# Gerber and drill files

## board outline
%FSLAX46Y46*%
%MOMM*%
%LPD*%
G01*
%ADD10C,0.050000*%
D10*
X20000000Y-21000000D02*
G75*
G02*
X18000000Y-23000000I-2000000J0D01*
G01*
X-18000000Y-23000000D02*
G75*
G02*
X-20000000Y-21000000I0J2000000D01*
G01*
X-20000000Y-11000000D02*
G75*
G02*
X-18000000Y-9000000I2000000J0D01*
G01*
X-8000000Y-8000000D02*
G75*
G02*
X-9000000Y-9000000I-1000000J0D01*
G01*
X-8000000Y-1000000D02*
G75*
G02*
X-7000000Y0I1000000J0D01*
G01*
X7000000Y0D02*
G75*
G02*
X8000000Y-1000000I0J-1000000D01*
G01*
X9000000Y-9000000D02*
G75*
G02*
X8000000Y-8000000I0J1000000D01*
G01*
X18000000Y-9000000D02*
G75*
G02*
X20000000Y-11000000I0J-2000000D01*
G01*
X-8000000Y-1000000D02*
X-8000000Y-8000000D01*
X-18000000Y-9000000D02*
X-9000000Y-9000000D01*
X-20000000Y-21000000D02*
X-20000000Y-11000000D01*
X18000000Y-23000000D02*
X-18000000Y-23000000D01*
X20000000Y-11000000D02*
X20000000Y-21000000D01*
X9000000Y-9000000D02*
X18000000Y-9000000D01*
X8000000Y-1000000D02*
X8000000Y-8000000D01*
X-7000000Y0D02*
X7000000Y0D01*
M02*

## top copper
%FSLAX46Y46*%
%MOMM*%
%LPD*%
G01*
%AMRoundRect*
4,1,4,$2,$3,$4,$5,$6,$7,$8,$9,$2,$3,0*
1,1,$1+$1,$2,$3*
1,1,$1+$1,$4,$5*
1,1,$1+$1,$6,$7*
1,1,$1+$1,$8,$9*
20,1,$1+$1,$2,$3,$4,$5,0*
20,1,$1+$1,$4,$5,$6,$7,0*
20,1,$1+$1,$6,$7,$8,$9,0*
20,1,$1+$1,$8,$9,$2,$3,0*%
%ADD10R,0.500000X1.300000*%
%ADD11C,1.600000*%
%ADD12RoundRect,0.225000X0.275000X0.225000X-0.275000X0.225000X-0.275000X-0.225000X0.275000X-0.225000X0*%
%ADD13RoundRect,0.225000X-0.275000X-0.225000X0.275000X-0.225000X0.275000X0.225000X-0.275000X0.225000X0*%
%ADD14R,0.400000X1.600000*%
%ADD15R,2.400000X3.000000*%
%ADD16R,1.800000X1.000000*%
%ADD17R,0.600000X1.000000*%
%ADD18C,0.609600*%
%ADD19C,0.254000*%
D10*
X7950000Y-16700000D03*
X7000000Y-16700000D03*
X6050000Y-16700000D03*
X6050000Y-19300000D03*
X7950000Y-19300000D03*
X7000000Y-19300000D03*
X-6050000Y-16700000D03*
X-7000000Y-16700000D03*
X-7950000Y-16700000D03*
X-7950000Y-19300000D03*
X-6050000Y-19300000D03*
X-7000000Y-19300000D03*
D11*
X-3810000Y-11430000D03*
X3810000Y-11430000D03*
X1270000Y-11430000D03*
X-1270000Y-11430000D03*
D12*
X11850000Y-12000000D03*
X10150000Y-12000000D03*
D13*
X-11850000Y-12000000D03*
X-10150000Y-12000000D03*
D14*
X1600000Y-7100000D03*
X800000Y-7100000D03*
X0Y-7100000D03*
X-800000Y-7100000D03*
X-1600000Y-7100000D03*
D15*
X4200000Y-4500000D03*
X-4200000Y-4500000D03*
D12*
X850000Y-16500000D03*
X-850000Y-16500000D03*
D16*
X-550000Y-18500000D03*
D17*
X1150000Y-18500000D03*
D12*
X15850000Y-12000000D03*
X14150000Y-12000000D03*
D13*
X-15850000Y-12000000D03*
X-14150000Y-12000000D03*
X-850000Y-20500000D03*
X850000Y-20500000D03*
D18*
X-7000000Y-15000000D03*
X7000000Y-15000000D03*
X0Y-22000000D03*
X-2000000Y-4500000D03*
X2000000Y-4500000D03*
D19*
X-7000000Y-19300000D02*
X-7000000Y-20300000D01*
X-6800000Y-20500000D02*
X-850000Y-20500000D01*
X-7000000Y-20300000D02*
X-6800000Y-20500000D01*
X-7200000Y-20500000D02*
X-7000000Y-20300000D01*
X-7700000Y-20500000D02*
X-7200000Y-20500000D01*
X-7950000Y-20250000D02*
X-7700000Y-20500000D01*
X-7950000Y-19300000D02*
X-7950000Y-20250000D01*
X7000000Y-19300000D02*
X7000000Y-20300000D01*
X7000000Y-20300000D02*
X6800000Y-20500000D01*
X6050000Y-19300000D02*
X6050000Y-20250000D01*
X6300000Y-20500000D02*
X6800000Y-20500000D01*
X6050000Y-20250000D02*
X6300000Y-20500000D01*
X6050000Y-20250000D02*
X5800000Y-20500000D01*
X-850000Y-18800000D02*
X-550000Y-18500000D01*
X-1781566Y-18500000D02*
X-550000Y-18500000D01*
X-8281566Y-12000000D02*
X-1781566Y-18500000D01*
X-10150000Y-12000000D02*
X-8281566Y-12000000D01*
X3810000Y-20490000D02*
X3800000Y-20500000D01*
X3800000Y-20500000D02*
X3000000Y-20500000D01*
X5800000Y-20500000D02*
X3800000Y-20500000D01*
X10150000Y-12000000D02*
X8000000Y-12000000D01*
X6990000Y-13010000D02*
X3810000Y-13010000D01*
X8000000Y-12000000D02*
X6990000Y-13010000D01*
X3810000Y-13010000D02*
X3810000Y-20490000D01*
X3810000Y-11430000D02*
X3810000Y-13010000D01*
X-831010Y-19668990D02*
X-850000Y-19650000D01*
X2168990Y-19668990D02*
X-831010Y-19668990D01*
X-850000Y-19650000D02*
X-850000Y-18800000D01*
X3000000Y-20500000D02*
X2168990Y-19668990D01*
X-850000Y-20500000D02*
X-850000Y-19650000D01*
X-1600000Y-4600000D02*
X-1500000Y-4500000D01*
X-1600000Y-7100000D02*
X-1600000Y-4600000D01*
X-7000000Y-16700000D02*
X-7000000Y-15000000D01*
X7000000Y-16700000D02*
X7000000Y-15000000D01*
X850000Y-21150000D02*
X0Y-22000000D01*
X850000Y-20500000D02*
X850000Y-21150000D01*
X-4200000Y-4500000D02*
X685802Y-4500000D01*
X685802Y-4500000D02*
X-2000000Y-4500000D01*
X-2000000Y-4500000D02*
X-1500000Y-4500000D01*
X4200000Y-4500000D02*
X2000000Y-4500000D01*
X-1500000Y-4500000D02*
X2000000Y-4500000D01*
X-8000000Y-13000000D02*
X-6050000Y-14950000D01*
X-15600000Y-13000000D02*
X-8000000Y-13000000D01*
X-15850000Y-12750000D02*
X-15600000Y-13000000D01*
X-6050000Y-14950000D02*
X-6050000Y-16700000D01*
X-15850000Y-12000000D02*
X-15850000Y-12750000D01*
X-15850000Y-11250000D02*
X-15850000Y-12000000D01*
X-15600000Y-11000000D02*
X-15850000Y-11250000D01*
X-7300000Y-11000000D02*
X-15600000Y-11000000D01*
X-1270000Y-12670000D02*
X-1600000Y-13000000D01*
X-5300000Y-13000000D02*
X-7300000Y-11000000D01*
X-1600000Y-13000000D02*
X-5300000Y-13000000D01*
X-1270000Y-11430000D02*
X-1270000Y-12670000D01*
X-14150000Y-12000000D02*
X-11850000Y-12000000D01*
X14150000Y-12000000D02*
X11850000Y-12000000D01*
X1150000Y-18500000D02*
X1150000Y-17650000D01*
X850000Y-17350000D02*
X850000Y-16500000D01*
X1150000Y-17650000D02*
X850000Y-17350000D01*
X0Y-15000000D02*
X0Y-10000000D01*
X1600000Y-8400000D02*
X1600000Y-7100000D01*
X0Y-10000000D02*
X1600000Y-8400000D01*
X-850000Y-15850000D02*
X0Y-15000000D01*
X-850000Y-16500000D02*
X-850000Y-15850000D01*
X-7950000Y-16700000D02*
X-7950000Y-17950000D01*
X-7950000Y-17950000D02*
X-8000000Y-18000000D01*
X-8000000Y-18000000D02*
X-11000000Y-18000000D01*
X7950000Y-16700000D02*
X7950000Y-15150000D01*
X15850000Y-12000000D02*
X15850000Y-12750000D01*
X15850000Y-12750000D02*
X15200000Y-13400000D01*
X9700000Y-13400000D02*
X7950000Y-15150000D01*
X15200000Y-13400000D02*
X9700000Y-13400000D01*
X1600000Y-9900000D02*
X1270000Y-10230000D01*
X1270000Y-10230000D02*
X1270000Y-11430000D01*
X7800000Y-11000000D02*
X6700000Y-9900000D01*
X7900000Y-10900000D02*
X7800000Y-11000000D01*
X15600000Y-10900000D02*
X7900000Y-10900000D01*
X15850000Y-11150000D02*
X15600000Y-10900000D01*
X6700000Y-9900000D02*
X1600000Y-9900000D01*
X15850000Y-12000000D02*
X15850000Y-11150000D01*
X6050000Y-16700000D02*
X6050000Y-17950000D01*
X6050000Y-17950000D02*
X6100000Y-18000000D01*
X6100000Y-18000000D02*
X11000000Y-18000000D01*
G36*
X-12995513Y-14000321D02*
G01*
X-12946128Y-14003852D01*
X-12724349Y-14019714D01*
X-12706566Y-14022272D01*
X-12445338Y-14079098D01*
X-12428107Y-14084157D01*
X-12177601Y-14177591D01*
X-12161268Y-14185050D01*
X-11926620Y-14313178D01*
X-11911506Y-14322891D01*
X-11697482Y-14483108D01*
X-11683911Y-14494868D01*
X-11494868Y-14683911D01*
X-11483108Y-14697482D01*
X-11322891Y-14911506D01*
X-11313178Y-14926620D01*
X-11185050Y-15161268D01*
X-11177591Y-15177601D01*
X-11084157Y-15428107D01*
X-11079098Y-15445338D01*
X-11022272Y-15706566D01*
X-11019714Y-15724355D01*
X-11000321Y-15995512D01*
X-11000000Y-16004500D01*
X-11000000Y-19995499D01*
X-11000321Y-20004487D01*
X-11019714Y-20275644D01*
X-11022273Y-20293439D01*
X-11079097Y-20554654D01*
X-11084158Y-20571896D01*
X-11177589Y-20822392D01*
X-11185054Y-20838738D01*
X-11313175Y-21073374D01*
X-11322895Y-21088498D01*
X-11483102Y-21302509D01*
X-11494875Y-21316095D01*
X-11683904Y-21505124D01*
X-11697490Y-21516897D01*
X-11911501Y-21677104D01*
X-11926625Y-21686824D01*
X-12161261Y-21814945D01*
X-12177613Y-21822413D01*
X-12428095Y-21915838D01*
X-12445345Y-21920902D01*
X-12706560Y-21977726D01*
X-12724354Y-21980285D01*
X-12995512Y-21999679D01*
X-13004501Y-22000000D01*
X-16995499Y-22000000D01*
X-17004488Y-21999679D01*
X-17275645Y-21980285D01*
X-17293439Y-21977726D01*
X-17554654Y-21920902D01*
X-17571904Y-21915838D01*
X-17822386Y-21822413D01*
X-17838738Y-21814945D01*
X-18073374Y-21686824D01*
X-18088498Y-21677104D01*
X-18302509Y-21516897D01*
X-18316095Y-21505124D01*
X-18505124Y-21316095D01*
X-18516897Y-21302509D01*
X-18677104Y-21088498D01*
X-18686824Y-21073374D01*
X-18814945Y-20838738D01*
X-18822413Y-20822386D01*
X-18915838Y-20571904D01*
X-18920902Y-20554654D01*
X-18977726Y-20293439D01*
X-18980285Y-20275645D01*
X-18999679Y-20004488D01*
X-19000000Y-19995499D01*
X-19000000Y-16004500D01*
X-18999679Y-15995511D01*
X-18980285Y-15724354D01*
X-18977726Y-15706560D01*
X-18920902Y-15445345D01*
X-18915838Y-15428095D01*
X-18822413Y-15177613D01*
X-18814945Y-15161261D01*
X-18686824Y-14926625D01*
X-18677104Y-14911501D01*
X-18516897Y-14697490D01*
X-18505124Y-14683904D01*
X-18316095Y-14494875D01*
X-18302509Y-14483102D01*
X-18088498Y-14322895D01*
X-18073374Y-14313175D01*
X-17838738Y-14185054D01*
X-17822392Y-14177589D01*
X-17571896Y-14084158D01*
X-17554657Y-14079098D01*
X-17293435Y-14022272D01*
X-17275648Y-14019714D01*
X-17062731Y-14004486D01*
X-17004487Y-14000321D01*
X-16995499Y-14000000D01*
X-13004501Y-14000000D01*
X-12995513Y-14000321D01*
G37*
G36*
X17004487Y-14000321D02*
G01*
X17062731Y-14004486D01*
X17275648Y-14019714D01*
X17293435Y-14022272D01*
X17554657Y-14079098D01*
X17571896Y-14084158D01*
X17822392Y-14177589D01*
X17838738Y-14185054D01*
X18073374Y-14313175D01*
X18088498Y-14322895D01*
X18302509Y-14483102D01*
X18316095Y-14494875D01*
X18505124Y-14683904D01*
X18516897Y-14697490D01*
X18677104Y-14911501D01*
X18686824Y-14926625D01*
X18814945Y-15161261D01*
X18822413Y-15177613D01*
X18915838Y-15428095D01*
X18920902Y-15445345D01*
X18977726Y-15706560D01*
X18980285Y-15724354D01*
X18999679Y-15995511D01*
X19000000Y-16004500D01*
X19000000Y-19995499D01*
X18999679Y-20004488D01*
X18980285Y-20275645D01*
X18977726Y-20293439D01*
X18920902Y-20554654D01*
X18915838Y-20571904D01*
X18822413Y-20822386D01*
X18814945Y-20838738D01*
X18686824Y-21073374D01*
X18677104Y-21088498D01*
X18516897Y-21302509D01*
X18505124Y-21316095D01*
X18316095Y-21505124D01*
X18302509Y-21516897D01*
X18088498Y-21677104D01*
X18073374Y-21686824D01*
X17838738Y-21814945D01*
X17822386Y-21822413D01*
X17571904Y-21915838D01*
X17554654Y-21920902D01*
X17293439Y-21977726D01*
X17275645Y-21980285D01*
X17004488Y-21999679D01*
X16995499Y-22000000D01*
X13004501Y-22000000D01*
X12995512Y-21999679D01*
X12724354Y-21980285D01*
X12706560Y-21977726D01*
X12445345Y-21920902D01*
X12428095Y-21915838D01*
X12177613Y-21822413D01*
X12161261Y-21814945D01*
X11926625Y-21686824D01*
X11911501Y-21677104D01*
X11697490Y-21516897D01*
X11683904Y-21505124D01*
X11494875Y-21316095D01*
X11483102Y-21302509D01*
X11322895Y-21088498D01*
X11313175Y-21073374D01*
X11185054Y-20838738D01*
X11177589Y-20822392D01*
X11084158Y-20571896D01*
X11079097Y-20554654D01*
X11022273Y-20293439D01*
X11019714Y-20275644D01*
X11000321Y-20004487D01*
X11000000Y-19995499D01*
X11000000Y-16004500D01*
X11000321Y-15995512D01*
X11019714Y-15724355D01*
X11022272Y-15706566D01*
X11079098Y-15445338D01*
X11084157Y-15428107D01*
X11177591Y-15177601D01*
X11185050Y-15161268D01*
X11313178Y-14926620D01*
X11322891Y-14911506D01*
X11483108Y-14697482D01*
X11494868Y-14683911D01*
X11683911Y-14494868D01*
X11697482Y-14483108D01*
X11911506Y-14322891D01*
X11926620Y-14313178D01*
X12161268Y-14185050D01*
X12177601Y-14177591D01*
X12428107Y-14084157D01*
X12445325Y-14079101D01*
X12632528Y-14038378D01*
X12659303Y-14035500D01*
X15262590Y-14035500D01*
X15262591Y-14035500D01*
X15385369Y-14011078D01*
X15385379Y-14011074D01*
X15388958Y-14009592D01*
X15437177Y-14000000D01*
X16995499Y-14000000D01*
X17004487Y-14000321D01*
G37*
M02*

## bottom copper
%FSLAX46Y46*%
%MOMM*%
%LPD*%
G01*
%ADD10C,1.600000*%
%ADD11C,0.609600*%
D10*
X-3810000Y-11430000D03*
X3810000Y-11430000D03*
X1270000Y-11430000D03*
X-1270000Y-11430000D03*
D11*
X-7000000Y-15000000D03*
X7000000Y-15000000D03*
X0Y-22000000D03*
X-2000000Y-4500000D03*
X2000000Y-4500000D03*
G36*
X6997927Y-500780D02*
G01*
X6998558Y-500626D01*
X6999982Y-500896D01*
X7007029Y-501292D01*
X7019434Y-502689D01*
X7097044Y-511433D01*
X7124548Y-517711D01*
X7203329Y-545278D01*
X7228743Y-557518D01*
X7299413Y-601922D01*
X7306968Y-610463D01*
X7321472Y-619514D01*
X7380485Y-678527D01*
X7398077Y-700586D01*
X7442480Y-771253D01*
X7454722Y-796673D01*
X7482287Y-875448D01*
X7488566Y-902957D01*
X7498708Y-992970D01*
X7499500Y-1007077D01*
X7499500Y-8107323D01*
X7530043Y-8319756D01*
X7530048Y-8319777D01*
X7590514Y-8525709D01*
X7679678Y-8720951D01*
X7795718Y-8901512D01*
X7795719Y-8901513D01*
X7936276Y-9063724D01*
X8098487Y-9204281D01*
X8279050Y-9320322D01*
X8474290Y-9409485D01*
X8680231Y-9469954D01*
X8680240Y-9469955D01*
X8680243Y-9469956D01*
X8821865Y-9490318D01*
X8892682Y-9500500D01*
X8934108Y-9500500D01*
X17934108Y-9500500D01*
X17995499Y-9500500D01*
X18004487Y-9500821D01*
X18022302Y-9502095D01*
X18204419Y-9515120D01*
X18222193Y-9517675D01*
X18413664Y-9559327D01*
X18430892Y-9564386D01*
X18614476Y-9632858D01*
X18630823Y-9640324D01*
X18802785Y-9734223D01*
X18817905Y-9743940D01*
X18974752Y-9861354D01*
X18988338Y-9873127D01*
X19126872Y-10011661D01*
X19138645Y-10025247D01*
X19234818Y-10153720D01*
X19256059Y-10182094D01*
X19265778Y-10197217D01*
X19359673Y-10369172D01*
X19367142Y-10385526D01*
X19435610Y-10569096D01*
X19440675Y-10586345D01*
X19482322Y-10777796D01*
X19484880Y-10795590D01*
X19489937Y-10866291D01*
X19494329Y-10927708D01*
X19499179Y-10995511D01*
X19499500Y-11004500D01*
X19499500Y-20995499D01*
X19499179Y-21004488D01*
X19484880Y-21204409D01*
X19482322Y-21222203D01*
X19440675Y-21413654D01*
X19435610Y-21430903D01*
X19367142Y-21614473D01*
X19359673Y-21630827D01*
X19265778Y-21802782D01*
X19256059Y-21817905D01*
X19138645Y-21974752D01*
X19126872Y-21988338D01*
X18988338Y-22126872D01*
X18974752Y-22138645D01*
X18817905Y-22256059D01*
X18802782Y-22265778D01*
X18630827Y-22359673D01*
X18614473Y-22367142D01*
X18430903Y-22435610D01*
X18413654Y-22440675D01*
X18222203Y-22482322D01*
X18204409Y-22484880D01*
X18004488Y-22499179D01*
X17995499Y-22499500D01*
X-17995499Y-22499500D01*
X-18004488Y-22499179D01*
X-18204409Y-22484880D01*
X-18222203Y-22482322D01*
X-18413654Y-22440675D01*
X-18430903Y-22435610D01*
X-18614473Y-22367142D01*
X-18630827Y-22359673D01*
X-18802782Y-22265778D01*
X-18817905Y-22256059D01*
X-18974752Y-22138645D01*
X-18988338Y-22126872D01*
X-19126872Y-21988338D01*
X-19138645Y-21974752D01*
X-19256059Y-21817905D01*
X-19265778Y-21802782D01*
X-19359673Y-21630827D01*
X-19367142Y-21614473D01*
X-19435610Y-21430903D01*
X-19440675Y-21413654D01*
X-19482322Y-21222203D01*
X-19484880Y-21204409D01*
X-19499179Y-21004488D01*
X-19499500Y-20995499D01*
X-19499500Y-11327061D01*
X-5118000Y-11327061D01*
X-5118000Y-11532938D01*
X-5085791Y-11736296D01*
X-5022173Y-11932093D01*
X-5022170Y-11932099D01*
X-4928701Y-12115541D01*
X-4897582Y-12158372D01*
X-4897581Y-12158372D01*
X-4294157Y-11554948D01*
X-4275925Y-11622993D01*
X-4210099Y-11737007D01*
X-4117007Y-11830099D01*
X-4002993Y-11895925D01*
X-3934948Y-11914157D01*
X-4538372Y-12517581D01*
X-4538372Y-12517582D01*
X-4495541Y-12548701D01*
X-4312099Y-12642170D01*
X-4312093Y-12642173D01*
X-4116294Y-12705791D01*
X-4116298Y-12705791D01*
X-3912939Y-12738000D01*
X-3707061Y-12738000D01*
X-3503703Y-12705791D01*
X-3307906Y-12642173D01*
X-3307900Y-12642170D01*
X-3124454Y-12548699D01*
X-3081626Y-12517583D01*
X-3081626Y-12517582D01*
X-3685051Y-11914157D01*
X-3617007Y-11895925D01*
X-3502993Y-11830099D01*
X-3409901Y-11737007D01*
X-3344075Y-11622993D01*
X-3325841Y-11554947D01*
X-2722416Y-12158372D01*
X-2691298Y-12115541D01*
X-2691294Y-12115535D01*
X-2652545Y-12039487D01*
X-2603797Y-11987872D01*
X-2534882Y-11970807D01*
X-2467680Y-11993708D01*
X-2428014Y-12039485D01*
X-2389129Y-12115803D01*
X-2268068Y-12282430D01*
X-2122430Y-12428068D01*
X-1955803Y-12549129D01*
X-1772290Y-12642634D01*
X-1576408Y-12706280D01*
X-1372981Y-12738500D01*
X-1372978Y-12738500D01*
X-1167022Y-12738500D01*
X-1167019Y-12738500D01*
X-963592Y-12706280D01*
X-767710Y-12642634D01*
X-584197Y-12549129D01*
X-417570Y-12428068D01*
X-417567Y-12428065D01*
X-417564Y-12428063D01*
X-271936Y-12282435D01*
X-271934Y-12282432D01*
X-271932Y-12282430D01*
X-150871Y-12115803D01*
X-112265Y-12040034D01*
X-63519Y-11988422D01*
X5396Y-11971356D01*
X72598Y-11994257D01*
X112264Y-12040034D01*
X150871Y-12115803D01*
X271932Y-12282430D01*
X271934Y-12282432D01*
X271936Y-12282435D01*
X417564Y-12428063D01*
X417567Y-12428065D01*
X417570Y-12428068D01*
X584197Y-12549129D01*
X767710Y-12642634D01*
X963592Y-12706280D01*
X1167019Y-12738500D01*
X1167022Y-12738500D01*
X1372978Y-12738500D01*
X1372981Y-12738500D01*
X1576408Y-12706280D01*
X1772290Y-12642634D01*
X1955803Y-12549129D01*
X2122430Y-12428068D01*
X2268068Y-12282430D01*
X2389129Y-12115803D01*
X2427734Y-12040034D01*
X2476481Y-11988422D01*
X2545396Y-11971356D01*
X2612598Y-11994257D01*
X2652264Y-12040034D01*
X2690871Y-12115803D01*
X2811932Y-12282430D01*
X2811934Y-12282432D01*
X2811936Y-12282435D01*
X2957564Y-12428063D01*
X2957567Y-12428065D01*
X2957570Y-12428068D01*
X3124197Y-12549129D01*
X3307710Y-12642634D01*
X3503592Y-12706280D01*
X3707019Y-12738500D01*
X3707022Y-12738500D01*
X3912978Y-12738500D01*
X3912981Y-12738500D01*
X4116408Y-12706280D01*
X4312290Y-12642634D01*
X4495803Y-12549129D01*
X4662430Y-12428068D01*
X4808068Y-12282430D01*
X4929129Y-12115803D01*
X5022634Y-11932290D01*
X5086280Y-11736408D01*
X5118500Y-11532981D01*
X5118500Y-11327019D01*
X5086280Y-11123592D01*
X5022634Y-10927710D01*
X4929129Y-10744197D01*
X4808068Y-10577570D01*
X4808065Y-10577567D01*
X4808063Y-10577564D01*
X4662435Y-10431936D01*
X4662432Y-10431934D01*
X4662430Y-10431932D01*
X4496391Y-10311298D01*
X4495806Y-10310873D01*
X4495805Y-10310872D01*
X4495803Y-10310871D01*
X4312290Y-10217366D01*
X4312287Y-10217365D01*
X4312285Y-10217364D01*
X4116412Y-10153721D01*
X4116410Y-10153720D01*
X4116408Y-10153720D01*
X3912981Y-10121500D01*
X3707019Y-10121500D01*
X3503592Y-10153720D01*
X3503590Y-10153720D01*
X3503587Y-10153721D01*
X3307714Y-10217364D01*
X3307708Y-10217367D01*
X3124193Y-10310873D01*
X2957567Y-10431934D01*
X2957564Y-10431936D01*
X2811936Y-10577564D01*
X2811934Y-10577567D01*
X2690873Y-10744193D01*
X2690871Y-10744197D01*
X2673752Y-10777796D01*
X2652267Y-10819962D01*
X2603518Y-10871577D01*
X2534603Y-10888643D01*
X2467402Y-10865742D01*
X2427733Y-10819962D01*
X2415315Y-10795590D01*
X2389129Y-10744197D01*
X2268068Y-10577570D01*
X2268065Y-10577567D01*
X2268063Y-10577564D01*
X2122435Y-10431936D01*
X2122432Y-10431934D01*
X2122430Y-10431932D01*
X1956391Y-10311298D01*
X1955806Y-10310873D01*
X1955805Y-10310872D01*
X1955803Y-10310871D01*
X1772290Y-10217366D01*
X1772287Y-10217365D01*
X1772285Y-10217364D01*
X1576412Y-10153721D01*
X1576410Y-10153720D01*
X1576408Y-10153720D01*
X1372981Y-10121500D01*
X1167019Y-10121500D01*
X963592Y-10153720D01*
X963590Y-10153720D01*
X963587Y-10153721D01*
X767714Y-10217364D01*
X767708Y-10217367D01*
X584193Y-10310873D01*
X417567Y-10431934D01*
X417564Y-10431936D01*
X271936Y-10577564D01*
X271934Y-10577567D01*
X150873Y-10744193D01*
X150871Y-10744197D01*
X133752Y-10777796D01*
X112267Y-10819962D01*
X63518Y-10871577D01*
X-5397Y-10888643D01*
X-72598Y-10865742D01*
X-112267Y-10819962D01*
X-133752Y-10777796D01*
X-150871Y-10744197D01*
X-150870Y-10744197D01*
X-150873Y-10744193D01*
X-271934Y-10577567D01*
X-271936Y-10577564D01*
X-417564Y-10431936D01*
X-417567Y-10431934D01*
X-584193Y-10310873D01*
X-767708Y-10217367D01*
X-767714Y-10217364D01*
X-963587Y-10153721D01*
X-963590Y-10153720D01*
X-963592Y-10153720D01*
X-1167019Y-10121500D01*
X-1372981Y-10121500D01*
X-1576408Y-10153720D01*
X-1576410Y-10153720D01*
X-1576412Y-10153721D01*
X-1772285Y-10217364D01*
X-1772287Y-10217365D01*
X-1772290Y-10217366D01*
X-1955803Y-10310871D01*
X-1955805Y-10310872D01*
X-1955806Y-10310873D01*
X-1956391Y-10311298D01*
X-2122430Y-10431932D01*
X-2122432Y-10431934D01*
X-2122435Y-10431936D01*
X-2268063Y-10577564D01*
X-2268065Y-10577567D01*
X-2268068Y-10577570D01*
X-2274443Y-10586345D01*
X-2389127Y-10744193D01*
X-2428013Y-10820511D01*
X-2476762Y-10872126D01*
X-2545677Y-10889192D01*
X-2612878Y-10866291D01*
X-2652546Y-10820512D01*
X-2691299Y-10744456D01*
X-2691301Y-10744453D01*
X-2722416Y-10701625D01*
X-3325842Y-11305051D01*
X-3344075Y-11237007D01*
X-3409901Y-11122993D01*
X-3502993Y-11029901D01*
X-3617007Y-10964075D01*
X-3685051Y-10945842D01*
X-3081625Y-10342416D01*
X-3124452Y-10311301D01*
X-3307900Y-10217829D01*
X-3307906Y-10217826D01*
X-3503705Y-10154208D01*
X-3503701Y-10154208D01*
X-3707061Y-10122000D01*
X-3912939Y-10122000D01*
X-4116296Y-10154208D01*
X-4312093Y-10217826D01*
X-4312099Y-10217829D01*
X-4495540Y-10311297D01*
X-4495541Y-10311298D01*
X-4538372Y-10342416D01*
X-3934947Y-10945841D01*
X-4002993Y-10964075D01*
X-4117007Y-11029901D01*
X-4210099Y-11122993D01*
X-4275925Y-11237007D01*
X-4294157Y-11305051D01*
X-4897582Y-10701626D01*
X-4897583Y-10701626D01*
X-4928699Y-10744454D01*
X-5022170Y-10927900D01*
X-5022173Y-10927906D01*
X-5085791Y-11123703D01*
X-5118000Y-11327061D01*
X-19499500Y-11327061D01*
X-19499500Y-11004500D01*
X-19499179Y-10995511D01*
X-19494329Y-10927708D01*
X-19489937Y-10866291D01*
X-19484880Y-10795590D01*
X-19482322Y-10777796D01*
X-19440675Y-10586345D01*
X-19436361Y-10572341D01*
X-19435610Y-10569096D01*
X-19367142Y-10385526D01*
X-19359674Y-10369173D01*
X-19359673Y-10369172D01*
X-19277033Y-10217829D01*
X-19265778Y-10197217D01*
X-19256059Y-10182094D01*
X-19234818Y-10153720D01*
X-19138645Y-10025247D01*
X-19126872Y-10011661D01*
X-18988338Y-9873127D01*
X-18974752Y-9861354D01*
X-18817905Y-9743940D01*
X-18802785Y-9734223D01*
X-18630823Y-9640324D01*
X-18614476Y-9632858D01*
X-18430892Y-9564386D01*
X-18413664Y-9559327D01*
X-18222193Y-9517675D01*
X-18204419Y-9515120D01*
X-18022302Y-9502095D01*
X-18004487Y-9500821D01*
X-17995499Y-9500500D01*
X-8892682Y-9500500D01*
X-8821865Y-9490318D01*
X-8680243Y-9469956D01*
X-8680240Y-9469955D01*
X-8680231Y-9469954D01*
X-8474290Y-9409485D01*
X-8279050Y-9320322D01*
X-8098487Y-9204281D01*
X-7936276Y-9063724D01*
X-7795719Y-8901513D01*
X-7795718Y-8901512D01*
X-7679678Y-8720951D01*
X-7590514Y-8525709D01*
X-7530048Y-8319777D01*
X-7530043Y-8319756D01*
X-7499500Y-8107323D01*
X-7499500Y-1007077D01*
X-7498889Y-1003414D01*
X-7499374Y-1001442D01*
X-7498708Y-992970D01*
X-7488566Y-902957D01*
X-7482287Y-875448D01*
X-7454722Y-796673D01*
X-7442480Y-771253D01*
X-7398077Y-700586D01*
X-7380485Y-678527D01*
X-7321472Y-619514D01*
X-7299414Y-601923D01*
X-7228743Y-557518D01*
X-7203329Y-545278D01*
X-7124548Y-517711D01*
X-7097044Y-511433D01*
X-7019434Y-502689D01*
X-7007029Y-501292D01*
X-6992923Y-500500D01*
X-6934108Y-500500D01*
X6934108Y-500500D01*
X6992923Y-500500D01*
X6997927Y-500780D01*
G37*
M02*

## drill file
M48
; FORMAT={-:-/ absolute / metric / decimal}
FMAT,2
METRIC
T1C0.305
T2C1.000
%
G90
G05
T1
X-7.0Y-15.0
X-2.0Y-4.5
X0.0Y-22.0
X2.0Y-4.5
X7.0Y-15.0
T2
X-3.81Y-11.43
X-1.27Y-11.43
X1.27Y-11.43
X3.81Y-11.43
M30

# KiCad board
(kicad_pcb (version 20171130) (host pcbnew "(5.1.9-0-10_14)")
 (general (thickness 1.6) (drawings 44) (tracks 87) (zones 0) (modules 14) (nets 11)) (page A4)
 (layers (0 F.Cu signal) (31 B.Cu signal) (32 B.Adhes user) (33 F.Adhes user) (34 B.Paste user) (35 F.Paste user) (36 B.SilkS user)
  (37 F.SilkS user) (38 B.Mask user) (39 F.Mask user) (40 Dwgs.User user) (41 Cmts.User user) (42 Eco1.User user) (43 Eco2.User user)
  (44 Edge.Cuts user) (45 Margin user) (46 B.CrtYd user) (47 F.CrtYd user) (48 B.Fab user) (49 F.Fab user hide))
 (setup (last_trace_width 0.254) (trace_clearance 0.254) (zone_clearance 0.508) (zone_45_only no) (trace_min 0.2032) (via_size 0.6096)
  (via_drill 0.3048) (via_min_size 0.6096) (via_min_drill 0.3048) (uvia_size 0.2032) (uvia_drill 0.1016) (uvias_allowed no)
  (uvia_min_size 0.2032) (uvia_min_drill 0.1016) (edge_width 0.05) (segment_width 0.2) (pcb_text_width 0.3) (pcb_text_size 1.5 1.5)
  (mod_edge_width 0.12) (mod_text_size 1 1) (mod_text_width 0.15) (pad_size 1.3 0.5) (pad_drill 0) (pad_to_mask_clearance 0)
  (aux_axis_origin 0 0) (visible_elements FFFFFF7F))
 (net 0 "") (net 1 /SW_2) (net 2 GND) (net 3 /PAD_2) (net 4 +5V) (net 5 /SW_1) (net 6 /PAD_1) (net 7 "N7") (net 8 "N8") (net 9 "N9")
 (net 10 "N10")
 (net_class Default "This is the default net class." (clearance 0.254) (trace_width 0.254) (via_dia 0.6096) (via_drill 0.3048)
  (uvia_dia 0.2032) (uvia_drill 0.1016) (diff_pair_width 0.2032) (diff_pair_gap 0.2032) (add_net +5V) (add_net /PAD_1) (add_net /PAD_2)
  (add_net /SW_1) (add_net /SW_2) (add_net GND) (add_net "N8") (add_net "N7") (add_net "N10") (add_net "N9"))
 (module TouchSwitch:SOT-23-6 (layer F.Cu) (at 7 18 270)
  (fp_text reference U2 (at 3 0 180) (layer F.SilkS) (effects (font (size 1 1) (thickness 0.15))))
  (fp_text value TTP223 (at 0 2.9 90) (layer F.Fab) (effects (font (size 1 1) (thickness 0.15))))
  (pad 1 smd rect (at -1.3 -0.95 270) (size 1.3 0.5) (layers F.Cu F.Paste F.Mask) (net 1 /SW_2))
  (pad 2 smd rect (at -1.3 0 270) (size 1.3 0.5) (layers F.Cu F.Paste F.Mask) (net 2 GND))
  (pad 3 smd rect (at -1.3 0.95 270) (size 1.3 0.5) (layers F.Cu F.Paste F.Mask) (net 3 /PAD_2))
  (pad 4 smd rect (at 1.3 0.95 270) (size 1.3 0.5) (layers F.Cu F.Paste F.Mask) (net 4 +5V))
  (pad 6 smd rect (at 1.3 -0.95 270) (size 1.3 0.5) (layers F.Cu F.Paste F.Mask))
  (pad 5 smd rect (at 1.3 0 270) (size 1.3 0.5) (layers F.Cu F.Paste F.Mask) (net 4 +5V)))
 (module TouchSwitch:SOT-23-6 (layer F.Cu) (at -7 18 270)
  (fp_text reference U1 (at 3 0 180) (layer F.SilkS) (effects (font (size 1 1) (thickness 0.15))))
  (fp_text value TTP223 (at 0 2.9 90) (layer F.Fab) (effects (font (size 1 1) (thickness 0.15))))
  (pad 1 smd rect (at -1.3 -0.95 270) (size 1.3 0.5) (layers F.Cu F.Paste F.Mask) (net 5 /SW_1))
  (pad 2 smd rect (at -1.3 0 270) (size 1.3 0.5) (layers F.Cu F.Paste F.Mask) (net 2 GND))
  (pad 3 smd rect (at -1.3 0.95 270) (size 1.3 0.5) (layers F.Cu F.Paste F.Mask) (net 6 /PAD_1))
  (pad 4 smd rect (at 1.3 0.95 270) (size 1.3 0.5) (layers F.Cu F.Paste F.Mask) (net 4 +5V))
  (pad 6 smd rect (at 1.3 -0.95 270) (size 1.3 0.5) (layers F.Cu F.Paste F.Mask))
  (pad 5 smd rect (at 1.3 0 270) (size 1.3 0.5) (layers F.Cu F.Paste F.Mask) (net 4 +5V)))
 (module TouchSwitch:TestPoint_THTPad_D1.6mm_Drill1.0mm (layer F.Cu) (at -3.81 11.43)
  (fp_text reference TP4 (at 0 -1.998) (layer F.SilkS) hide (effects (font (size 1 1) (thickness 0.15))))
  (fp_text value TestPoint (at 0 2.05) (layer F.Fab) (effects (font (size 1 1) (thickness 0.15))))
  (pad 1 thru_hole circle (at 0 0) (size 1.6 1.6) (drill 1) (layers *.Cu *.Mask) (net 2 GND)))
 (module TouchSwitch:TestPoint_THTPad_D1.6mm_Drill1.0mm (layer F.Cu) (at 3.81 11.43)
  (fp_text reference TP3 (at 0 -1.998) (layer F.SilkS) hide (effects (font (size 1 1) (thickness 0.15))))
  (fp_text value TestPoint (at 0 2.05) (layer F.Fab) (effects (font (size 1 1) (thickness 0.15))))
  (pad 1 thru_hole circle (at 0 0) (size 1.6 1.6) (drill 1) (layers *.Cu *.Mask) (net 4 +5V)))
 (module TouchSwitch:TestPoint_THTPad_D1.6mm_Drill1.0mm (layer F.Cu) (at 1.27 11.43)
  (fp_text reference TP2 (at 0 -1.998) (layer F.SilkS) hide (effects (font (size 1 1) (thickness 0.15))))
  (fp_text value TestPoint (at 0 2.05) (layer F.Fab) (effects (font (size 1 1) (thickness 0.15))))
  (pad 1 thru_hole circle (at 0 0) (size 1.6 1.6) (drill 1) (layers *.Cu *.Mask) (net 1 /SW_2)))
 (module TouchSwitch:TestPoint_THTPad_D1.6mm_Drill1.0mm (layer F.Cu) (at -1.27 11.43)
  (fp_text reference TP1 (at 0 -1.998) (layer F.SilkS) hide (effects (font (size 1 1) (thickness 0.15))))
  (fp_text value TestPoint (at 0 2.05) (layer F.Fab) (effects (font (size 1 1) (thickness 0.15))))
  (pad 1 thru_hole circle (at 0 0) (size 1.6 1.6) (drill 1) (layers *.Cu *.Mask) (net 5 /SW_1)))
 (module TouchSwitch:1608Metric (layer F.Cu) (at 11 12 180)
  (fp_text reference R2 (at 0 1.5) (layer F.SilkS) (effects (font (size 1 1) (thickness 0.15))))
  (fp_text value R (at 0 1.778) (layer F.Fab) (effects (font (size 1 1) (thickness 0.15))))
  (pad 1 smd roundrect (at -0.85 0 180) (size 1 0.9) (layers F.Cu F.Paste F.Mask) (roundrect_rratio 0.25) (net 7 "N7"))
  (pad 2 smd roundrect (at 0.85 0 180) (size 1 0.9) (layers F.Cu F.Paste F.Mask) (roundrect_rratio 0.25) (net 4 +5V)))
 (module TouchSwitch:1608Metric (layer F.Cu) (at -11 12)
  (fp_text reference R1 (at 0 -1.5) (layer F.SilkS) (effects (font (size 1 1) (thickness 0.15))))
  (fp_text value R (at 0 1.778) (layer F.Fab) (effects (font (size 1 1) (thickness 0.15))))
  (pad 1 smd roundrect (at -0.85 0) (size 1 0.9) (layers F.Cu F.Paste F.Mask) (roundrect_rratio 0.25) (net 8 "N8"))
  (pad 2 smd roundrect (at 0.85 0) (size 1 0.9) (layers F.Cu F.Paste F.Mask) (roundrect_rratio 0.25) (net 4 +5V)))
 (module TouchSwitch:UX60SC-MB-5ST (layer F.Cu) (at 0 0 180)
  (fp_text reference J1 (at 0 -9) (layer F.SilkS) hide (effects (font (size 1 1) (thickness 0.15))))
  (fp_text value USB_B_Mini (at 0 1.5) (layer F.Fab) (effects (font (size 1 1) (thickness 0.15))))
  (pad 1 smd rect (at -1.6 -7.1 180) (size 0.4 1.6) (layers F.Cu F.Paste F.Mask) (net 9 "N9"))
  (pad 2 smd rect (at -0.8 -7.1 180) (size 0.4 1.6) (layers F.Cu F.Paste F.Mask))
  (pad 3 smd rect (at 0 -7.1 180) (size 0.4 1.6) (layers F.Cu F.Paste F.Mask))
  (pad 4 smd rect (at 0.8 -7.1 180) (size 0.4 1.6) (layers F.Cu F.Paste F.Mask))
  (pad 5 smd rect (at 1.6 -7.1 180) (size 0.4 1.6) (layers F.Cu F.Paste F.Mask) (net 2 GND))
  (pad 6 smd rect (at -4.2 -4.5) (size 2.4 3) (layers F.Cu F.Paste F.Mask) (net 2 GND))
  (pad 6 smd rect (at 4.2 -4.5) (size 2.4 3) (layers F.Cu F.Paste F.Mask) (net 2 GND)))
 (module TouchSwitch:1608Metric (layer F.Cu) (at 0 16.5 180)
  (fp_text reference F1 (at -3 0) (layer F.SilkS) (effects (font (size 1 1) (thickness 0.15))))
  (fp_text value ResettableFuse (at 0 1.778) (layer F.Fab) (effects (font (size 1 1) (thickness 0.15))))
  (pad 1 smd roundrect (at -0.85 0 180) (size 1 0.9) (layers F.Cu F.Paste F.Mask) (roundrect_rratio 0.25) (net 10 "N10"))
  (pad 2 smd roundrect (at 0.85 0 180) (size 1 0.9) (layers F.Cu F.Paste F.Mask) (roundrect_rratio 0.25) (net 9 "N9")))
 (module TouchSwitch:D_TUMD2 (layer F.Cu) (at 0 18.5)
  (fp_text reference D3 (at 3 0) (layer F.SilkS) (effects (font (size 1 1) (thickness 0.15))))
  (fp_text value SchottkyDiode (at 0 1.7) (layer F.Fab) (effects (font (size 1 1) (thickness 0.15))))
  (pad 1 smd rect (at -0.55 0 180) (size 1.8 1) (layers F.Cu F.Paste F.Mask) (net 4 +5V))
  (pad 2 smd rect (at 1.15 0 180) (size 0.6 1) (layers F.Cu F.Paste F.Mask) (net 10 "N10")))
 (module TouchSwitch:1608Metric (layer F.Cu) (at 15 12 180)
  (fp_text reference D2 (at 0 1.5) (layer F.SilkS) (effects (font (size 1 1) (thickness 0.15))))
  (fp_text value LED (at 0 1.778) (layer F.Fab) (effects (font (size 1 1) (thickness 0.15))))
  (pad 1 smd roundrect (at -0.85 0 180) (size 1 0.9) (layers F.Cu F.Paste F.Mask) (roundrect_rratio 0.25) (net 1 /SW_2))
  (pad 2 smd roundrect (at 0.85 0 180) (size 1 0.9) (layers F.Cu F.Paste F.Mask) (roundrect_rratio 0.25) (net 7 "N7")))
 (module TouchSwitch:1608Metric (layer F.Cu) (at -15 12)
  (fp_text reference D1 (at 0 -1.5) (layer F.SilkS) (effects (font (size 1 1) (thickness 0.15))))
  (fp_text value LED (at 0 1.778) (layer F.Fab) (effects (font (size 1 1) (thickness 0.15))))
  (pad 1 smd roundrect (at -0.85 0) (size 1 0.9) (layers F.Cu F.Paste F.Mask) (roundrect_rratio 0.25) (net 5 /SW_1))
  (pad 2 smd roundrect (at 0.85 0) (size 1 0.9) (layers F.Cu F.Paste F.Mask) (roundrect_rratio 0.25) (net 8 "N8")))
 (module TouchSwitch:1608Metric (layer F.Cu) (at 0 20.5)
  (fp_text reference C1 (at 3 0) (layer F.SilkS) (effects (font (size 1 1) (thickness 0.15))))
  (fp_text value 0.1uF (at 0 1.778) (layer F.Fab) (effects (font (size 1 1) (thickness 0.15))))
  (pad 1 smd roundrect (at -0.85 0) (size 1 0.9) (layers F.Cu F.Paste F.Mask) (roundrect_rratio 0.25) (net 4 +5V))
  (pad 2 smd roundrect (at 0.85 0) (size 1 0.9) (layers F.Cu F.Paste F.Mask) (roundrect_rratio 0.25) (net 2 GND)))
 (gr_arc (start 18 21) (end 18 23) (angle -90) (layer Edge.Cuts) (width 0.05))
 (gr_arc (start -18 21) (end -20 21) (angle -90) (layer Edge.Cuts) (width 0.05))
 (gr_arc (start -18 11) (end -18 9) (angle -90) (layer Edge.Cuts) (width 0.05))
 (gr_arc (start -9 8) (end -9 9) (angle -90) (layer Edge.Cuts) (width 0.05))
 (gr_arc (start -7 1) (end -7 0) (angle -90) (layer Edge.Cuts) (width 0.05))
 (gr_arc (start 7 1) (end 8 1) (angle -90) (layer Edge.Cuts) (width 0.05))
 (gr_arc (start 9 8) (end 8 8) (angle -90) (layer Edge.Cuts) (width 0.05))
 (gr_arc (start 18 11) (end 20 11) (angle -90) (layer Edge.Cuts) (width 0.05))
 (gr_line (start -8 1) (end -8 8) (layer Edge.Cuts) (width 0.05))
 (gr_line (start -18 9) (end -9 9) (layer Edge.Cuts) (width 0.05))
 (gr_line (start -20 21) (end -20 11) (layer Edge.Cuts) (width 0.05))
 (gr_line (start 18 23) (end -18 23) (layer Edge.Cuts) (width 0.05))
 (gr_line (start 20 11) (end 20 21) (layer Edge.Cuts) (width 0.05))
 (gr_line (start 9 9) (end 18 9) (layer Edge.Cuts) (width 0.05))
 (gr_line (start 8 1) (end 8 8) (layer Edge.Cuts) (width 0.05))
 (gr_line (start -7 0) (end 7 0) (layer Edge.Cuts) (width 0.05))
 (segment (start -7 19.3) (end -7 20.3) (width 0.254) (layer F.Cu) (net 4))
 (segment (start -6.8 20.5) (end -0.85 20.5) (width 0.254) (layer F.Cu) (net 4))
 (segment (start -7 20.3) (end -6.8 20.5) (width 0.254) (layer F.Cu) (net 4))
 (segment (start -7.2 20.5) (end -7 20.3) (width 0.254) (layer F.Cu) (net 4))
 (segment (start -7.7 20.5) (end -7.2 20.5) (width 0.254) (layer F.Cu) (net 4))
 (segment (start -7.95 20.25) (end -7.7 20.5) (width 0.254) (layer F.Cu) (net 4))
 (segment (start -7.95 19.3) (end -7.95 20.25) (width 0.254) (layer F.Cu) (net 4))
 (segment (start 7 19.3) (end 7 20.3) (width 0.254) (layer F.Cu) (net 4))
 (segment (start 7 20.3) (end 6.8 20.5) (width 0.254) (layer F.Cu) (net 4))
 (segment (start 6.05 19.3) (end 6.05 20.25) (width 0.254) (layer F.Cu) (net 4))
 (segment (start 6.3 20.5) (end 6.8 20.5) (width 0.254) (layer F.Cu) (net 4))
 (segment (start 6.05 20.25) (end 6.3 20.5) (width 0.254) (layer F.Cu) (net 4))
 (segment (start 6.05 20.25) (end 5.8 20.5) (width 0.254) (layer F.Cu) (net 4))
 (segment (start -0.85 18.8) (end -0.55 18.5) (width 0.254) (layer F.Cu) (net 4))
 (segment (start -1.781566 18.5) (end -0.55 18.5) (width 0.254) (layer F.Cu) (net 4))
 (segment (start -8.281566 12) (end -1.781566 18.5) (width 0.254) (layer F.Cu) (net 4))
 (segment (start -10.15 12) (end -8.281566 12) (width 0.254) (layer F.Cu) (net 4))
 (segment (start 3.81 20.49) (end 3.8 20.5) (width 0.254) (layer F.Cu) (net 4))
 (segment (start 3.8 20.5) (end 3 20.5) (width 0.254) (layer F.Cu) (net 4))
 (segment (start 5.8 20.5) (end 3.8 20.5) (width 0.254) (layer F.Cu) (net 4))
 (segment (start 10.15 12) (end 8 12) (width 0.254) (layer F.Cu) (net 4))
 (segment (start 6.99 13.01) (end 3.81 13.01) (width 0.254) (layer F.Cu) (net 4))
 (segment (start 8 12) (end 6.99 13.01) (width 0.254) (layer F.Cu) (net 4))
 (segment (start 3.81 13.01) (end 3.81 20.49) (width 0.254) (layer F.Cu) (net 4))
 (segment (start 3.81 11.43) (end 3.81 13.01) (width 0.254) (layer F.Cu) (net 4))
 (segment (start -0.83101 19.66899) (end -0.85 19.65) (width 0.254) (layer F.Cu) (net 4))
 (segment (start 2.16899 19.66899) (end -0.83101 19.66899) (width 0.254) (layer F.Cu) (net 4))
 (segment (start -0.85 19.65) (end -0.85 18.8) (width 0.254) (layer F.Cu) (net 4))
 (segment (start 3 20.5) (end 2.16899 19.66899) (width 0.254) (layer F.Cu) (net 4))
 (segment (start -0.85 20.5) (end -0.85 19.65) (width 0.254) (layer F.Cu) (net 4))
 (segment (start -1.6 4.6) (end -1.5 4.5) (width 0.254) (layer F.Cu) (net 2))
 (segment (start -1.6 7.1) (end -1.6 4.6) (width 0.254) (layer F.Cu) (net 2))
 (via (at -7 15) (size 0.6096) (drill 0.3048) (layers F.Cu B.Cu) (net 2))
 (segment (start -7 16.7) (end -7 15) (width 0.254) (layer F.Cu) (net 2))
 (via (at 7 15) (size 0.6096) (drill 0.3048) (layers F.Cu B.Cu) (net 2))
 (segment (start 7 16.7) (end 7 15) (width 0.254) (layer F.Cu) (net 2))
 (via (at 0 22) (size 0.6096) (drill 0.3048) (layers F.Cu B.Cu) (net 2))
 (segment (start 0.85 21.15) (end 0 22) (width 0.254) (layer F.Cu) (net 2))
 (segment (start 0.85 20.5) (end 0.85 21.15) (width 0.254) (layer F.Cu) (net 2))
 (via (at -2 4.5) (size 0.6096) (drill 0.3048) (layers F.Cu B.Cu) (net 2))
 (segment (start -4.2 4.5) (end 0.685802 4.5) (width 0.254) (layer F.Cu) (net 2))
 (segment (start 0.685802 4.5) (end -2 4.5) (width 0.254) (layer F.Cu) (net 2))
 (segment (start -2 4.5) (end -1.5 4.5) (width 0.254) (layer F.Cu) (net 2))
 (via (at 2 4.5) (size 0.6096) (drill 0.3048) (layers F.Cu B.Cu) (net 2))
 (segment (start 4.2 4.5) (end 2 4.5) (width 0.254) (layer F.Cu) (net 2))
 (segment (start -1.5 4.5) (end 2 4.5) (width 0.254) (layer F.Cu) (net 2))
 (segment (start -8 13) (end -6.05 14.95) (width 0.254) (layer F.Cu) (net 5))
 (segment (start -15.6 13) (end -8 13) (width 0.254) (layer F.Cu) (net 5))
 (segment (start -15.85 12.75) (end -15.6 13) (width 0.254) (layer F.Cu) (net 5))
 (segment (start -6.05 14.95) (end -6.05 16.7) (width 0.254) (layer F.Cu) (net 5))
 (segment (start -15.85 12) (end -15.85 12.75) (width 0.254) (layer F.Cu) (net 5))
 (segment (start -15.85 11.25) (end -15.85 12) (width 0.254) (layer F.Cu) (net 5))
 (segment (start -15.6 11) (end -15.85 11.25) (width 0.254) (layer F.Cu) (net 5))
 (segment (start -7.3 11) (end -15.6 11) (width 0.254) (layer F.Cu) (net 5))
 (segment (start -1.27 12.67) (end -1.6 13) (width 0.254) (layer F.Cu) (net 5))
 (segment (start -5.3 13) (end -7.3 11) (width 0.254) (layer F.Cu) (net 5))
 (segment (start -1.6 13) (end -5.3 13) (width 0.254) (layer F.Cu) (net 5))
 (segment (start -1.27 11.43) (end -1.27 12.67) (width 0.254) (layer F.Cu) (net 5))
 (segment (start -14.15 12) (end -11.85 12) (width 0.254) (layer F.Cu) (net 8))
 (segment (start 14.15 12) (end 11.85 12) (width 0.254) (layer F.Cu) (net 7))
 (segment (start 1.15 18.5) (end 1.15 17.65) (width 0.254) (layer F.Cu) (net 10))
 (segment (start 0.85 17.35) (end 0.85 16.5) (width 0.254) (layer F.Cu) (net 10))
 (segment (start 1.15 17.65) (end 0.85 17.35) (width 0.254) (layer F.Cu) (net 10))
 (segment (start 0 15) (end 0 10) (width 0.254) (layer F.Cu) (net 9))
 (segment (start 1.6 8.4) (end 1.6 7.1) (width 0.254) (layer F.Cu) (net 9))
 (segment (start 0 10) (end 1.6 8.4) (width 0.254) (layer F.Cu) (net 9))
 (segment (start -0.85 15.85) (end 0 15) (width 0.254) (layer F.Cu) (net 9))
 (segment (start -0.85 16.5) (end -0.85 15.85) (width 0.254) (layer F.Cu) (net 9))
 (segment (start -7.95 16.7) (end -7.95 17.95) (width 0.254) (layer F.Cu) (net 6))
 (segment (start -7.95 17.95) (end -8 18) (width 0.254) (layer F.Cu) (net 6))
 (segment (start -8 18) (end -11 18) (width 0.254) (layer F.Cu) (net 6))
 (segment (start 7.95 16.7) (end 7.95 15.15) (width 0.254) (layer F.Cu) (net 1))
 (segment (start 15.85 12) (end 15.85 12.75) (width 0.254) (layer F.Cu) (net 1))
 (segment (start 15.85 12.75) (end 15.2 13.4) (width 0.254) (layer F.Cu) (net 1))
 (segment (start 9.7 13.4) (end 7.95 15.15) (width 0.254) (layer F.Cu) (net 1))
 (segment (start 15.2 13.4) (end 9.7 13.4) (width 0.254) (layer F.Cu) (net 1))
 (segment (start 1.6 9.9) (end 1.27 10.23) (width 0.254) (layer F.Cu) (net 1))
 (segment (start 1.27 10.23) (end 1.27 11.43) (width 0.254) (layer F.Cu) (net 1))
 (segment (start 7.8 11) (end 6.7 9.9) (width 0.254) (layer F.Cu) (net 1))
 (segment (start 7.9 10.9) (end 7.8 11) (width 0.254) (layer F.Cu) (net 1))
 (segment (start 15.6 10.9) (end 7.9 10.9) (width 0.254) (layer F.Cu) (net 1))
 (segment (start 15.85 11.15) (end 15.6 10.9) (width 0.254) (layer F.Cu) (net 1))
 (segment (start 6.7 9.9) (end 1.6 9.9) (width 0.254) (layer F.Cu) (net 1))
 (segment (start 15.85 12) (end 15.85 11.15) (width 0.254) (layer F.Cu) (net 1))
 (segment (start 6.05 16.7) (end 6.05 17.95) (width 0.254) (layer F.Cu) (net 3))
 (segment (start 6.05 17.95) (end 6.1 18) (width 0.254) (layer F.Cu) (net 3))
 (segment (start 6.1 18) (end 11 18) (width 0.254) (layer F.Cu) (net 3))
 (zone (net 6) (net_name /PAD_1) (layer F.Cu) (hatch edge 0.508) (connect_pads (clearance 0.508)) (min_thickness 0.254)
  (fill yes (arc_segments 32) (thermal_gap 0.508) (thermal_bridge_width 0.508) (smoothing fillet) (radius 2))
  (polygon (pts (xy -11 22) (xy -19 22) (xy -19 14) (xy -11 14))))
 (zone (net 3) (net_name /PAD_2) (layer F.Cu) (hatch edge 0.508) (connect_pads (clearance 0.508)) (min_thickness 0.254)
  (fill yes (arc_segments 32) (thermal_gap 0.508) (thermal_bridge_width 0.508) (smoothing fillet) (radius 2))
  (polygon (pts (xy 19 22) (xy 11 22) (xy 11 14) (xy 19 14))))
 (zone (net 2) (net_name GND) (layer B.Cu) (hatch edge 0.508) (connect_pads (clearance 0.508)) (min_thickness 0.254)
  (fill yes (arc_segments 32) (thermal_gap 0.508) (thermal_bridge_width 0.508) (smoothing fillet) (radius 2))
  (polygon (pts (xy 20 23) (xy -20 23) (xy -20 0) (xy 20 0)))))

